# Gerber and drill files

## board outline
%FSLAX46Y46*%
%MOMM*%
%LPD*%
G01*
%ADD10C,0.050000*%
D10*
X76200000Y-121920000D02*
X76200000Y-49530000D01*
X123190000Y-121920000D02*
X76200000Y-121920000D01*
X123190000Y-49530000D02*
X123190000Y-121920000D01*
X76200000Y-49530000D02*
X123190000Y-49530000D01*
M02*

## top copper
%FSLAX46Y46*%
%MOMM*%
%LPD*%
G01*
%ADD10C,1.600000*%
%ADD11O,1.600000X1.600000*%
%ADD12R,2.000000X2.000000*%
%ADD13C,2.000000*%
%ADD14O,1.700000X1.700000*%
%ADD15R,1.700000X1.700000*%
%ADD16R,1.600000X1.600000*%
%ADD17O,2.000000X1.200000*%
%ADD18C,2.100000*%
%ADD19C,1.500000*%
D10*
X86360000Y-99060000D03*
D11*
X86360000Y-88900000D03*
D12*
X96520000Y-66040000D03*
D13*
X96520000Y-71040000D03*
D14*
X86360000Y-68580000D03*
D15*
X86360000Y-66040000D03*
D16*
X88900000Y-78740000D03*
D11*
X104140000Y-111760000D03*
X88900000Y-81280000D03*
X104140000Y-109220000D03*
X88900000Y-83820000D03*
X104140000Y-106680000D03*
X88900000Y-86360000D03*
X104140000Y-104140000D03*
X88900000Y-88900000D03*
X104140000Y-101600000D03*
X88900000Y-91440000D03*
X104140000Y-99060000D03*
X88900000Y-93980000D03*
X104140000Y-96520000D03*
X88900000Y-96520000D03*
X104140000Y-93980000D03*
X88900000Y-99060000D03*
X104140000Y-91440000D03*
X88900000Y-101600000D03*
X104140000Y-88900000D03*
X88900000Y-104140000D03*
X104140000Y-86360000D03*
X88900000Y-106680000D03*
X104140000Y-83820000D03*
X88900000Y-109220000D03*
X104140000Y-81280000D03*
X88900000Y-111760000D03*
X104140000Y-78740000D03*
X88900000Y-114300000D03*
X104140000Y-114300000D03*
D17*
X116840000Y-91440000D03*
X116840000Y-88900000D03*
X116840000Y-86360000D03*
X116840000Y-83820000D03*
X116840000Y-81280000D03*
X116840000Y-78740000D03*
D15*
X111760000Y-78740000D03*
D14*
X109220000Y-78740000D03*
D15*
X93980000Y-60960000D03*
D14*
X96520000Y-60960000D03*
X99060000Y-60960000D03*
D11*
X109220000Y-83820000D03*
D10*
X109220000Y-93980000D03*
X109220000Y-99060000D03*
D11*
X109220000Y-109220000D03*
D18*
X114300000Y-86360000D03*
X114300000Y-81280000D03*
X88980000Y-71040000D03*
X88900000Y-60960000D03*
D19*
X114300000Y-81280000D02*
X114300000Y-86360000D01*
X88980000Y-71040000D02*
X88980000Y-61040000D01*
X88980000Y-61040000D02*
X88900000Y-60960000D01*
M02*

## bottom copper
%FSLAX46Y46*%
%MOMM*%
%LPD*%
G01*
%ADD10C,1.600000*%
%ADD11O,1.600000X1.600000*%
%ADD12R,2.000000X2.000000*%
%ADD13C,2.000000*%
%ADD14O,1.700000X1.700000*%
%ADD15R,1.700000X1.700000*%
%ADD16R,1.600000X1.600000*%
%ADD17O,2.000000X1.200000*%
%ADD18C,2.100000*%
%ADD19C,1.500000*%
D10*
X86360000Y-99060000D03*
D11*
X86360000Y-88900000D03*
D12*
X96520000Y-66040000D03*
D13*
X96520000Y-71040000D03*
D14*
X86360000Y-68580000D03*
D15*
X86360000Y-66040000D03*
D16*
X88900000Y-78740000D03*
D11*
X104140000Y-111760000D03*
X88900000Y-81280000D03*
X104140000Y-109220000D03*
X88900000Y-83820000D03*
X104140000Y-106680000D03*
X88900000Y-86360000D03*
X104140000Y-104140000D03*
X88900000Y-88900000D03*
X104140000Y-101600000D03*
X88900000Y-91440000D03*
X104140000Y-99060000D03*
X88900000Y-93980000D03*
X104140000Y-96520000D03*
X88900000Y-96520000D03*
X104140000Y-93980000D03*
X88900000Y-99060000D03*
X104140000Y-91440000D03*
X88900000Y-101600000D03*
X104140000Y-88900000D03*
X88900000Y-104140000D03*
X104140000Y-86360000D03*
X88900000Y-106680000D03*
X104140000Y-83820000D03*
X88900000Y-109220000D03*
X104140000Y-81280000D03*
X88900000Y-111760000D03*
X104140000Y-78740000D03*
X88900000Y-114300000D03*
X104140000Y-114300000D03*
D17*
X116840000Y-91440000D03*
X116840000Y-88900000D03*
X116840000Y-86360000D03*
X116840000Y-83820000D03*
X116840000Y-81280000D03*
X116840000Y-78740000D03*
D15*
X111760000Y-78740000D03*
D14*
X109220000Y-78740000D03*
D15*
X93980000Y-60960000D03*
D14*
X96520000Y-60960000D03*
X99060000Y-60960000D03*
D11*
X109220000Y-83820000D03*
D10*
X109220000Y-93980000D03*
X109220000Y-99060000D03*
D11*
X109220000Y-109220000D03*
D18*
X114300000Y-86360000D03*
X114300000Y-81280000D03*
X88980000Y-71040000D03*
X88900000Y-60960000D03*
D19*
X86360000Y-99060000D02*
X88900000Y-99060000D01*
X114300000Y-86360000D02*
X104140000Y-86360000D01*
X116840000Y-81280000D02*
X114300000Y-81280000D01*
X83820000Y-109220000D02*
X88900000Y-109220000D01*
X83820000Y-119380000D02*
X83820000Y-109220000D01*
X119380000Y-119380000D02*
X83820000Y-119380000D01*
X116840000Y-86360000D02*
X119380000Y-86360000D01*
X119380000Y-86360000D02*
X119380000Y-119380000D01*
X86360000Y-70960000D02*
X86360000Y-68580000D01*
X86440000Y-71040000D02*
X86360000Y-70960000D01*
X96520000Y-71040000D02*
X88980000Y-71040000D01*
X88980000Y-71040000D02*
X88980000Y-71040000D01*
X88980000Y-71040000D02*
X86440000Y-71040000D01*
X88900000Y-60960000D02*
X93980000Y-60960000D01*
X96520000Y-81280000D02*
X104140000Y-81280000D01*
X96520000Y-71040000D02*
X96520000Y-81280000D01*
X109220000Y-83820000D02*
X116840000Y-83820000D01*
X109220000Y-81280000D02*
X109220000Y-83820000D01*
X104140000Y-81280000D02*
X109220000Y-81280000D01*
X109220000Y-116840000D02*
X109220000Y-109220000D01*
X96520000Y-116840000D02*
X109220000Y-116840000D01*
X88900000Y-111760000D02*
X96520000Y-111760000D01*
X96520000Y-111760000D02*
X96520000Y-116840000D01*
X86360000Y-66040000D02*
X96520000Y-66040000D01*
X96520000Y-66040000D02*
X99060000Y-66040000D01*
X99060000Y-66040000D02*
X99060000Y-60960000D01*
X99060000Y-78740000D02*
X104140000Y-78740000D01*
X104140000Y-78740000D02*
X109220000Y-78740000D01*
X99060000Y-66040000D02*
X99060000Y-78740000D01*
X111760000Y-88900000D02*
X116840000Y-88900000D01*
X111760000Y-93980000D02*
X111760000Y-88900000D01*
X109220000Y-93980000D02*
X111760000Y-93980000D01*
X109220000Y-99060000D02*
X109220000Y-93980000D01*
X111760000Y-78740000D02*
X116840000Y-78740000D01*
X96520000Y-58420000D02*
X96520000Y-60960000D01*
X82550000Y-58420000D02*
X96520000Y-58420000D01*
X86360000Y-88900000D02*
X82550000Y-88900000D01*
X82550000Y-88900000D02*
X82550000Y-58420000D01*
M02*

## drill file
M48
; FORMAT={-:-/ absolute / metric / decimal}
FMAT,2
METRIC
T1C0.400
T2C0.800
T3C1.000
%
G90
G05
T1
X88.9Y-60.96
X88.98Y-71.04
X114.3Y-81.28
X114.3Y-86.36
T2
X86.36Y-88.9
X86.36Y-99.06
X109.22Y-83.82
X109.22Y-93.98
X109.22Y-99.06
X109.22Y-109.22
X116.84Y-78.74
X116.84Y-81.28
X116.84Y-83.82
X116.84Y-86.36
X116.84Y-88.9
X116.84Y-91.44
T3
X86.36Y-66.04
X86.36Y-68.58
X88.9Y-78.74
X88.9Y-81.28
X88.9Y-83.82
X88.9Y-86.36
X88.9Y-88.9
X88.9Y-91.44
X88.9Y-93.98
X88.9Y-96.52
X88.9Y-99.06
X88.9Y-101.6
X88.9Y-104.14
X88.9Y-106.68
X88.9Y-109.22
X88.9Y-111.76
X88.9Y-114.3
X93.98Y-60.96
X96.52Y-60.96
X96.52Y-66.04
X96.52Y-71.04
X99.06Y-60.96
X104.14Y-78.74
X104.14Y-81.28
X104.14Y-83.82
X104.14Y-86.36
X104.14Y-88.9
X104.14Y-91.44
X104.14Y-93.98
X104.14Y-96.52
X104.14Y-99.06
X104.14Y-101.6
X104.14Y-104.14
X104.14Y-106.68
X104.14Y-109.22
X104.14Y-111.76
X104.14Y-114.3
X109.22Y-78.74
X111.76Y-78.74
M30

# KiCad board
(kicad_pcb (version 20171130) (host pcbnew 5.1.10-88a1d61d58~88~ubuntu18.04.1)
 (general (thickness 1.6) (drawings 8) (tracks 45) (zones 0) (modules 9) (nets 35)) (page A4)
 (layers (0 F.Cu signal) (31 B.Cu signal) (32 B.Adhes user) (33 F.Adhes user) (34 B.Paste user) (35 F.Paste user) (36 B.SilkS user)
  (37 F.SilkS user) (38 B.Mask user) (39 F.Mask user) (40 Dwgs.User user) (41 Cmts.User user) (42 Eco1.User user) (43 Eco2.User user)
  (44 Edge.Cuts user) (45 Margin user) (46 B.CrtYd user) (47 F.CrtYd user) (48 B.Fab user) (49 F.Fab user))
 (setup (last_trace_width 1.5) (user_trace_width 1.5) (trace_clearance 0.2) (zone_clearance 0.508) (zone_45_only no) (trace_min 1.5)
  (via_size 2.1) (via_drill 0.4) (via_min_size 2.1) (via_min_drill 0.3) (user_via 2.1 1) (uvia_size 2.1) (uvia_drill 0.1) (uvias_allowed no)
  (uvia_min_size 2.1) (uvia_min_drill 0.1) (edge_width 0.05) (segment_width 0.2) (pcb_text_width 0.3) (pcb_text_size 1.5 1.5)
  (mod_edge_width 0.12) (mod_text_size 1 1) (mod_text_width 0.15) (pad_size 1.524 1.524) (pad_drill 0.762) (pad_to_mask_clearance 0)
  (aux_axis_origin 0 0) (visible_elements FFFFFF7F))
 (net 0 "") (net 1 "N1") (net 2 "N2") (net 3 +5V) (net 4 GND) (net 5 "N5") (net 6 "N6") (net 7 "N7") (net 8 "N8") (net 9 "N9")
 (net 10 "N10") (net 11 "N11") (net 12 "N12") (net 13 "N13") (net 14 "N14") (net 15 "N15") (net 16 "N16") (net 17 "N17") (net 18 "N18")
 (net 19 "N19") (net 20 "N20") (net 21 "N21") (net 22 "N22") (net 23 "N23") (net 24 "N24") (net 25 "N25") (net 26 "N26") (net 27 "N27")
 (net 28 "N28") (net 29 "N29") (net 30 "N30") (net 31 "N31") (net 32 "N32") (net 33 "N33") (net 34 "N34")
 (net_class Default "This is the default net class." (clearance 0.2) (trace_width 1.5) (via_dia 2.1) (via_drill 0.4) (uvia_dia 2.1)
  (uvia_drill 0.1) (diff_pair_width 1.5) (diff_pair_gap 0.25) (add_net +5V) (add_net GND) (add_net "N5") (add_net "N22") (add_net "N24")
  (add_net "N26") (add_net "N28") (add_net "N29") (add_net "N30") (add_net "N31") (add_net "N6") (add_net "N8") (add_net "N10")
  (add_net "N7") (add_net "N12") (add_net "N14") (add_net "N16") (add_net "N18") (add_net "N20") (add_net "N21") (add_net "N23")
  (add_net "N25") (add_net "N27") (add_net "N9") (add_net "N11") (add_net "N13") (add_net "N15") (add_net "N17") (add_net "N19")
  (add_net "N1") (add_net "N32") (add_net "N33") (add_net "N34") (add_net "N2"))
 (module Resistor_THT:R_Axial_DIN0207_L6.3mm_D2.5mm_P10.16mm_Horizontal (layer F.Cu) (at 86.36 99.06 90)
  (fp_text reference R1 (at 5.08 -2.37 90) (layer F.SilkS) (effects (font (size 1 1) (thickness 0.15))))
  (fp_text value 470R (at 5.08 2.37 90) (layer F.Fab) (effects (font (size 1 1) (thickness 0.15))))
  (pad 1 thru_hole circle (at 0 0 90) (size 1.6 1.6) (drill 0.8) (layers *.Cu *.Mask) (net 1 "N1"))
  (pad 2 thru_hole oval (at 10.16 0 90) (size 1.6 1.6) (drill 0.8) (layers *.Cu *.Mask) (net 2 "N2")))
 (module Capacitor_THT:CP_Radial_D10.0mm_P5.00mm (layer F.Cu) (at 96.52 66.04 270)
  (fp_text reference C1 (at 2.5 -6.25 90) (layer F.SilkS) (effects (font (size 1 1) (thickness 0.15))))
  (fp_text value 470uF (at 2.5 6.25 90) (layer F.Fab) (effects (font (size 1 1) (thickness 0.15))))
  (pad 1 thru_hole rect (at 0 0 270) (size 2 2) (drill 1) (layers *.Cu *.Mask) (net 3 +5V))
  (pad 2 thru_hole circle (at 5 0 270) (size 2 2) (drill 1) (layers *.Cu *.Mask) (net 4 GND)))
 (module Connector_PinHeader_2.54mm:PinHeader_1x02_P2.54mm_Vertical (layer F.Cu) (at 86.36 66.04)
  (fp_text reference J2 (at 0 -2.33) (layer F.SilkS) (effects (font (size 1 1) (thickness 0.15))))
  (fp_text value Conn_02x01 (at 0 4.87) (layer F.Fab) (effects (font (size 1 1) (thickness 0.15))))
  (pad 2 thru_hole oval (at 0 2.54) (size 1.7 1.7) (drill 1) (layers *.Cu *.Mask) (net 4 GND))
  (pad 1 thru_hole rect (at 0 0) (size 1.7 1.7) (drill 1) (layers *.Cu *.Mask) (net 3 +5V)))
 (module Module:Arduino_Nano (layer F.Cu) (at 88.9 78.74)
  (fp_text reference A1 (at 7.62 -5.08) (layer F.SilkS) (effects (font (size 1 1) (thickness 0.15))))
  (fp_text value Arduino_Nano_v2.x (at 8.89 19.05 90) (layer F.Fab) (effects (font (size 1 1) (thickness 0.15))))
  (pad 1 thru_hole rect (at 0 0) (size 1.6 1.6) (drill 1) (layers *.Cu *.Mask) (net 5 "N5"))
  (pad 17 thru_hole oval (at 15.24 33.02) (size 1.6 1.6) (drill 1) (layers *.Cu *.Mask) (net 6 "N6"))
  (pad 2 thru_hole oval (at 0 2.54) (size 1.6 1.6) (drill 1) (layers *.Cu *.Mask) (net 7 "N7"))
  (pad 18 thru_hole oval (at 15.24 30.48) (size 1.6 1.6) (drill 1) (layers *.Cu *.Mask) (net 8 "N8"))
  (pad 3 thru_hole oval (at 0 5.08) (size 1.6 1.6) (drill 1) (layers *.Cu *.Mask) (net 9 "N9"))
  (pad 19 thru_hole oval (at 15.24 27.94) (size 1.6 1.6) (drill 1) (layers *.Cu *.Mask) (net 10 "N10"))
  (pad 4 thru_hole oval (at 0 7.62) (size 1.6 1.6) (drill 1) (layers *.Cu *.Mask) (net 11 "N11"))
  (pad 20 thru_hole oval (at 15.24 25.4) (size 1.6 1.6) (drill 1) (layers *.Cu *.Mask) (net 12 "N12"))
  (pad 5 thru_hole oval (at 0 10.16) (size 1.6 1.6) (drill 1) (layers *.Cu *.Mask) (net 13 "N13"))
  (pad 21 thru_hole oval (at 15.24 22.86) (size 1.6 1.6) (drill 1) (layers *.Cu *.Mask) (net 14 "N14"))
  (pad 6 thru_hole oval (at 0 12.7) (size 1.6 1.6) (drill 1) (layers *.Cu *.Mask) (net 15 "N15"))
  (pad 22 thru_hole oval (at 15.24 20.32) (size 1.6 1.6) (drill 1) (layers *.Cu *.Mask) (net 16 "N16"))
  (pad 7 thru_hole oval (at 0 15.24) (size 1.6 1.6) (drill 1) (layers *.Cu *.Mask) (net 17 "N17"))
  (pad 23 thru_hole oval (at 15.24 17.78) (size 1.6 1.6) (drill 1) (layers *.Cu *.Mask) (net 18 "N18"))
  (pad 8 thru_hole oval (at 0 17.78) (size 1.6 1.6) (drill 1) (layers *.Cu *.Mask) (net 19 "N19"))
  (pad 24 thru_hole oval (at 15.24 15.24) (size 1.6 1.6) (drill 1) (layers *.Cu *.Mask) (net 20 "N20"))
  (pad 9 thru_hole oval (at 0 20.32) (size 1.6 1.6) (drill 1) (layers *.Cu *.Mask) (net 1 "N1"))
  (pad 25 thru_hole oval (at 15.24 12.7) (size 1.6 1.6) (drill 1) (layers *.Cu *.Mask) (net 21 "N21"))
  (pad 10 thru_hole oval (at 0 22.86) (size 1.6 1.6) (drill 1) (layers *.Cu *.Mask) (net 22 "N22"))
  (pad 26 thru_hole oval (at 15.24 10.16) (size 1.6 1.6) (drill 1) (layers *.Cu *.Mask) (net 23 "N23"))
  (pad 11 thru_hole oval (at 0 25.4) (size 1.6 1.6) (drill 1) (layers *.Cu *.Mask) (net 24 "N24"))
  (pad 27 thru_hole oval (at 15.24 7.62) (size 1.6 1.6) (drill 1) (layers *.Cu *.Mask) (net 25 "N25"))
  (pad 12 thru_hole oval (at 0 27.94) (size 1.6 1.6) (drill 1) (layers *.Cu *.Mask) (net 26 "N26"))
  (pad 28 thru_hole oval (at 15.24 5.08) (size 1.6 1.6) (drill 1) (layers *.Cu *.Mask) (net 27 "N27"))
  (pad 13 thru_hole oval (at 0 30.48) (size 1.6 1.6) (drill 1) (layers *.Cu *.Mask) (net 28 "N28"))
  (pad 29 thru_hole oval (at 15.24 2.54) (size 1.6 1.6) (drill 1) (layers *.Cu *.Mask) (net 4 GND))
  (pad 14 thru_hole oval (at 0 33.02) (size 1.6 1.6) (drill 1) (layers *.Cu *.Mask) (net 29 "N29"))
  (pad 30 thru_hole oval (at 15.24 0) (size 1.6 1.6) (drill 1) (layers *.Cu *.Mask) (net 3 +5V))
  (pad 15 thru_hole oval (at 0 35.56) (size 1.6 1.6) (drill 1) (layers *.Cu *.Mask) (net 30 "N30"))
  (pad 16 thru_hole oval (at 15.24 35.56) (size 1.6 1.6) (drill 1) (layers *.Cu *.Mask) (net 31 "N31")))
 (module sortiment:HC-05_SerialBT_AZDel (layer F.Cu) (at 116.84 85.09 90)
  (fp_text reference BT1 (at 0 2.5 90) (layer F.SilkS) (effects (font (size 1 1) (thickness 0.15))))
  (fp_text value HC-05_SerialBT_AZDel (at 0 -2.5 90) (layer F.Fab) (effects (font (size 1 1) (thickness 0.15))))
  (pad 1 thru_hole oval (at -6.35 0 90) (size 1.2 2) (drill 0.8) (layers *.Cu *.Mask) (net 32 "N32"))
  (pad 2 thru_hole oval (at -3.81 0 90) (size 1.2 2) (drill 0.8) (layers *.Cu *.Mask) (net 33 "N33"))
  (pad 3 thru_hole oval (at -1.27 0 90) (size 1.2 2) (drill 0.8) (layers *.Cu *.Mask) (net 28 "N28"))
  (pad 4 thru_hole oval (at 1.27 0 90) (size 1.2 2) (drill 0.8) (layers *.Cu *.Mask) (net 4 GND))
  (pad 5 thru_hole oval (at 3.81 0 90) (size 1.2 2) (drill 0.8) (layers *.Cu *.Mask) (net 25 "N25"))
  (pad 6 thru_hole oval (at 6.35 0 90) (size 1.2 2) (drill 0.8) (layers *.Cu *.Mask) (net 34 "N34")))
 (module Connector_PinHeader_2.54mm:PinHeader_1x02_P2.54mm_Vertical (layer F.Cu) (at 111.76 78.74 270)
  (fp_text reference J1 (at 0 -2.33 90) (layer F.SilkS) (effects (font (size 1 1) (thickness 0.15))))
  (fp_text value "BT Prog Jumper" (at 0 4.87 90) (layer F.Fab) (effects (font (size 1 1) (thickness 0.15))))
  (pad 1 thru_hole rect (at 0 0 270) (size 1.7 1.7) (drill 1) (layers *.Cu *.Mask) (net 34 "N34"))
  (pad 2 thru_hole oval (at 0 2.54 270) (size 1.7 1.7) (drill 1) (layers *.Cu *.Mask) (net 3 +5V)))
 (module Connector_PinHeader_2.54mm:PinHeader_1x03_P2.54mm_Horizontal (layer F.Cu) (at 93.98 60.96 90)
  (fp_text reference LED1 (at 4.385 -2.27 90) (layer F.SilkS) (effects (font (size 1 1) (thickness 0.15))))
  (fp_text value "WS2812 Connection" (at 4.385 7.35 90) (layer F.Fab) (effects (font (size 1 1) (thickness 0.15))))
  (pad 1 thru_hole rect (at 0 0 90) (size 1.7 1.7) (drill 1) (layers *.Cu *.Mask) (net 4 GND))
  (pad 2 thru_hole oval (at 0 2.54 90) (size 1.7 1.7) (drill 1) (layers *.Cu *.Mask) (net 2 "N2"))
  (pad 3 thru_hole oval (at 0 5.08 90) (size 1.7 1.7) (drill 1) (layers *.Cu *.Mask) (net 3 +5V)))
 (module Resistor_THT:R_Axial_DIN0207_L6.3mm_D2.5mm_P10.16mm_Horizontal (layer F.Cu) (at 109.22 93.98 90)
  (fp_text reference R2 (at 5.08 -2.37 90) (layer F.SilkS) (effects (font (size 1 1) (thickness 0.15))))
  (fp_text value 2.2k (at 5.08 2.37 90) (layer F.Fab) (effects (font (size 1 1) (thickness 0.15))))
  (pad 2 thru_hole oval (at 10.16 0 90) (size 1.6 1.6) (drill 0.8) (layers *.Cu *.Mask) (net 4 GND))
  (pad 1 thru_hole circle (at 0 0 90) (size 1.6 1.6) (drill 0.8) (layers *.Cu *.Mask) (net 33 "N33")))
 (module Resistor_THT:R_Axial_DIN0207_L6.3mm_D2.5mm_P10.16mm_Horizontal (layer F.Cu) (at 109.22 99.06 270)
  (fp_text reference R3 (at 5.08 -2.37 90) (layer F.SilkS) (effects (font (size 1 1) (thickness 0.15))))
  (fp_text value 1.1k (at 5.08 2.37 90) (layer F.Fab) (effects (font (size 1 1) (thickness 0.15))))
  (pad 1 thru_hole circle (at 0 0 270) (size 1.6 1.6) (drill 0.8) (layers *.Cu *.Mask) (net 33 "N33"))
  (pad 2 thru_hole oval (at 10.16 0 270) (size 1.6 1.6) (drill 0.8) (layers *.Cu *.Mask) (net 29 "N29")))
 (gr_line (start 76.2 121.92) (end 76.2 49.53) (layer Edge.Cuts) (width 0.05))
 (gr_line (start 123.19 121.92) (end 76.2 121.92) (layer Edge.Cuts) (width 0.05))
 (gr_line (start 123.19 49.53) (end 123.19 121.92) (layer Edge.Cuts) (width 0.05))
 (gr_line (start 76.2 49.53) (end 123.19 49.53) (layer Edge.Cuts) (width 0.05))
 (segment (start 86.36 99.06) (end 88.9 99.06) (width 1.5) (layer B.Cu) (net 1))
 (via (at 114.3 86.36) (size 2.1) (drill 0.4) (layers F.Cu B.Cu) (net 25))
 (segment (start 114.3 86.36) (end 104.14 86.36) (width 1.5) (layer B.Cu) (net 25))
 (segment (start 114.3 81.28) (end 114.3 86.36) (width 1.5) (layer F.Cu) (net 25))
 (via (at 114.3 81.28) (size 2.1) (drill 0.4) (layers F.Cu B.Cu) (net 25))
 (segment (start 116.84 81.28) (end 114.3 81.28) (width 1.5) (layer B.Cu) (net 25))
 (segment (start 83.82 109.22) (end 88.9 109.22) (width 1.5) (layer B.Cu) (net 28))
 (segment (start 83.82 119.38) (end 83.82 109.22) (width 1.5) (layer B.Cu) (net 28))
 (segment (start 119.38 119.38) (end 83.82 119.38) (width 1.5) (layer B.Cu) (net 28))
 (segment (start 116.84 86.36) (end 119.38 86.36) (width 1.5) (layer B.Cu) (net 28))
 (segment (start 119.38 86.36) (end 119.38 119.38) (width 1.5) (layer B.Cu) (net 28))
 (segment (start 86.36 70.96) (end 86.36 68.58) (width 1.5) (layer B.Cu) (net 4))
 (segment (start 86.44 71.04) (end 86.36 70.96) (width 1.5) (layer B.Cu) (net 4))
 (segment (start 96.52 71.04) (end 88.98 71.04) (width 1.5) (layer B.Cu) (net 4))
 (segment (start 88.98 71.04) (end 88.98 71.04) (width 1.5) (layer B.Cu) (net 4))
 (segment (start 88.98 71.04) (end 86.44 71.04) (width 1.5) (layer B.Cu) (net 4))
 (via (at 88.98 71.04) (size 2.1) (drill 0.4) (layers F.Cu B.Cu) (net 4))
 (via (at 88.9 60.96) (size 2.1) (drill 0.4) (layers F.Cu B.Cu) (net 4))
 (segment (start 88.98 71.04) (end 88.98 61.04) (width 1.5) (layer F.Cu) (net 4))
 (segment (start 88.98 61.04) (end 88.9 60.96) (width 1.5) (layer F.Cu) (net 4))
 (segment (start 88.9 60.96) (end 93.98 60.96) (width 1.5) (layer B.Cu) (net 4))
 (segment (start 96.52 81.28) (end 104.14 81.28) (width 1.5) (layer B.Cu) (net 4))
 (segment (start 96.52 71.04) (end 96.52 81.28) (width 1.5) (layer B.Cu) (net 4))
 (segment (start 109.22 83.82) (end 116.84 83.82) (width 1.5) (layer B.Cu) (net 4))
 (segment (start 109.22 81.28) (end 109.22 83.82) (width 1.5) (layer B.Cu) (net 4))
 (segment (start 104.14 81.28) (end 109.22 81.28) (width 1.5) (layer B.Cu) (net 4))
 (segment (start 109.22 116.84) (end 109.22 109.22) (width 1.5) (layer B.Cu) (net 29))
 (segment (start 96.52 116.84) (end 109.22 116.84) (width 1.5) (layer B.Cu) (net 29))
 (segment (start 88.9 111.76) (end 96.52 111.76) (width 1.5) (layer B.Cu) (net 29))
 (segment (start 96.52 111.76) (end 96.52 116.84) (width 1.5) (layer B.Cu) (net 29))
 (segment (start 86.36 66.04) (end 96.52 66.04) (width 1.5) (layer B.Cu) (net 3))
 (segment (start 96.52 66.04) (end 99.06 66.04) (width 1.5) (layer B.Cu) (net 3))
 (segment (start 99.06 66.04) (end 99.06 60.96) (width 1.5) (layer B.Cu) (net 3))
 (segment (start 99.06 78.74) (end 104.14 78.74) (width 1.5) (layer B.Cu) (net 3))
 (segment (start 104.14 78.74) (end 109.22 78.74) (width 1.5) (layer B.Cu) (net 3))
 (segment (start 99.06 66.04) (end 99.06 78.74) (width 1.5) (layer B.Cu) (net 3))
 (segment (start 111.76 88.9) (end 116.84 88.9) (width 1.5) (layer B.Cu) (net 33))
 (segment (start 111.76 93.98) (end 111.76 88.9) (width 1.5) (layer B.Cu) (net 33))
 (segment (start 109.22 93.98) (end 111.76 93.98) (width 1.5) (layer B.Cu) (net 33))
 (segment (start 109.22 99.06) (end 109.22 93.98) (width 1.5) (layer B.Cu) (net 33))
 (segment (start 111.76 78.74) (end 116.84 78.74) (width 1.5) (layer B.Cu) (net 34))
 (segment (start 96.52 58.42) (end 96.52 60.96) (width 1.5) (layer B.Cu) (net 2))
 (segment (start 82.55 58.42) (end 96.52 58.42) (width 1.5) (layer B.Cu) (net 2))
 (segment (start 86.36 88.9) (end 82.55 88.9) (width 1.5) (layer B.Cu) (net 2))
 (segment (start 82.55 88.9) (end 82.55 58.42) (width 1.5) (layer B.Cu) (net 2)))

